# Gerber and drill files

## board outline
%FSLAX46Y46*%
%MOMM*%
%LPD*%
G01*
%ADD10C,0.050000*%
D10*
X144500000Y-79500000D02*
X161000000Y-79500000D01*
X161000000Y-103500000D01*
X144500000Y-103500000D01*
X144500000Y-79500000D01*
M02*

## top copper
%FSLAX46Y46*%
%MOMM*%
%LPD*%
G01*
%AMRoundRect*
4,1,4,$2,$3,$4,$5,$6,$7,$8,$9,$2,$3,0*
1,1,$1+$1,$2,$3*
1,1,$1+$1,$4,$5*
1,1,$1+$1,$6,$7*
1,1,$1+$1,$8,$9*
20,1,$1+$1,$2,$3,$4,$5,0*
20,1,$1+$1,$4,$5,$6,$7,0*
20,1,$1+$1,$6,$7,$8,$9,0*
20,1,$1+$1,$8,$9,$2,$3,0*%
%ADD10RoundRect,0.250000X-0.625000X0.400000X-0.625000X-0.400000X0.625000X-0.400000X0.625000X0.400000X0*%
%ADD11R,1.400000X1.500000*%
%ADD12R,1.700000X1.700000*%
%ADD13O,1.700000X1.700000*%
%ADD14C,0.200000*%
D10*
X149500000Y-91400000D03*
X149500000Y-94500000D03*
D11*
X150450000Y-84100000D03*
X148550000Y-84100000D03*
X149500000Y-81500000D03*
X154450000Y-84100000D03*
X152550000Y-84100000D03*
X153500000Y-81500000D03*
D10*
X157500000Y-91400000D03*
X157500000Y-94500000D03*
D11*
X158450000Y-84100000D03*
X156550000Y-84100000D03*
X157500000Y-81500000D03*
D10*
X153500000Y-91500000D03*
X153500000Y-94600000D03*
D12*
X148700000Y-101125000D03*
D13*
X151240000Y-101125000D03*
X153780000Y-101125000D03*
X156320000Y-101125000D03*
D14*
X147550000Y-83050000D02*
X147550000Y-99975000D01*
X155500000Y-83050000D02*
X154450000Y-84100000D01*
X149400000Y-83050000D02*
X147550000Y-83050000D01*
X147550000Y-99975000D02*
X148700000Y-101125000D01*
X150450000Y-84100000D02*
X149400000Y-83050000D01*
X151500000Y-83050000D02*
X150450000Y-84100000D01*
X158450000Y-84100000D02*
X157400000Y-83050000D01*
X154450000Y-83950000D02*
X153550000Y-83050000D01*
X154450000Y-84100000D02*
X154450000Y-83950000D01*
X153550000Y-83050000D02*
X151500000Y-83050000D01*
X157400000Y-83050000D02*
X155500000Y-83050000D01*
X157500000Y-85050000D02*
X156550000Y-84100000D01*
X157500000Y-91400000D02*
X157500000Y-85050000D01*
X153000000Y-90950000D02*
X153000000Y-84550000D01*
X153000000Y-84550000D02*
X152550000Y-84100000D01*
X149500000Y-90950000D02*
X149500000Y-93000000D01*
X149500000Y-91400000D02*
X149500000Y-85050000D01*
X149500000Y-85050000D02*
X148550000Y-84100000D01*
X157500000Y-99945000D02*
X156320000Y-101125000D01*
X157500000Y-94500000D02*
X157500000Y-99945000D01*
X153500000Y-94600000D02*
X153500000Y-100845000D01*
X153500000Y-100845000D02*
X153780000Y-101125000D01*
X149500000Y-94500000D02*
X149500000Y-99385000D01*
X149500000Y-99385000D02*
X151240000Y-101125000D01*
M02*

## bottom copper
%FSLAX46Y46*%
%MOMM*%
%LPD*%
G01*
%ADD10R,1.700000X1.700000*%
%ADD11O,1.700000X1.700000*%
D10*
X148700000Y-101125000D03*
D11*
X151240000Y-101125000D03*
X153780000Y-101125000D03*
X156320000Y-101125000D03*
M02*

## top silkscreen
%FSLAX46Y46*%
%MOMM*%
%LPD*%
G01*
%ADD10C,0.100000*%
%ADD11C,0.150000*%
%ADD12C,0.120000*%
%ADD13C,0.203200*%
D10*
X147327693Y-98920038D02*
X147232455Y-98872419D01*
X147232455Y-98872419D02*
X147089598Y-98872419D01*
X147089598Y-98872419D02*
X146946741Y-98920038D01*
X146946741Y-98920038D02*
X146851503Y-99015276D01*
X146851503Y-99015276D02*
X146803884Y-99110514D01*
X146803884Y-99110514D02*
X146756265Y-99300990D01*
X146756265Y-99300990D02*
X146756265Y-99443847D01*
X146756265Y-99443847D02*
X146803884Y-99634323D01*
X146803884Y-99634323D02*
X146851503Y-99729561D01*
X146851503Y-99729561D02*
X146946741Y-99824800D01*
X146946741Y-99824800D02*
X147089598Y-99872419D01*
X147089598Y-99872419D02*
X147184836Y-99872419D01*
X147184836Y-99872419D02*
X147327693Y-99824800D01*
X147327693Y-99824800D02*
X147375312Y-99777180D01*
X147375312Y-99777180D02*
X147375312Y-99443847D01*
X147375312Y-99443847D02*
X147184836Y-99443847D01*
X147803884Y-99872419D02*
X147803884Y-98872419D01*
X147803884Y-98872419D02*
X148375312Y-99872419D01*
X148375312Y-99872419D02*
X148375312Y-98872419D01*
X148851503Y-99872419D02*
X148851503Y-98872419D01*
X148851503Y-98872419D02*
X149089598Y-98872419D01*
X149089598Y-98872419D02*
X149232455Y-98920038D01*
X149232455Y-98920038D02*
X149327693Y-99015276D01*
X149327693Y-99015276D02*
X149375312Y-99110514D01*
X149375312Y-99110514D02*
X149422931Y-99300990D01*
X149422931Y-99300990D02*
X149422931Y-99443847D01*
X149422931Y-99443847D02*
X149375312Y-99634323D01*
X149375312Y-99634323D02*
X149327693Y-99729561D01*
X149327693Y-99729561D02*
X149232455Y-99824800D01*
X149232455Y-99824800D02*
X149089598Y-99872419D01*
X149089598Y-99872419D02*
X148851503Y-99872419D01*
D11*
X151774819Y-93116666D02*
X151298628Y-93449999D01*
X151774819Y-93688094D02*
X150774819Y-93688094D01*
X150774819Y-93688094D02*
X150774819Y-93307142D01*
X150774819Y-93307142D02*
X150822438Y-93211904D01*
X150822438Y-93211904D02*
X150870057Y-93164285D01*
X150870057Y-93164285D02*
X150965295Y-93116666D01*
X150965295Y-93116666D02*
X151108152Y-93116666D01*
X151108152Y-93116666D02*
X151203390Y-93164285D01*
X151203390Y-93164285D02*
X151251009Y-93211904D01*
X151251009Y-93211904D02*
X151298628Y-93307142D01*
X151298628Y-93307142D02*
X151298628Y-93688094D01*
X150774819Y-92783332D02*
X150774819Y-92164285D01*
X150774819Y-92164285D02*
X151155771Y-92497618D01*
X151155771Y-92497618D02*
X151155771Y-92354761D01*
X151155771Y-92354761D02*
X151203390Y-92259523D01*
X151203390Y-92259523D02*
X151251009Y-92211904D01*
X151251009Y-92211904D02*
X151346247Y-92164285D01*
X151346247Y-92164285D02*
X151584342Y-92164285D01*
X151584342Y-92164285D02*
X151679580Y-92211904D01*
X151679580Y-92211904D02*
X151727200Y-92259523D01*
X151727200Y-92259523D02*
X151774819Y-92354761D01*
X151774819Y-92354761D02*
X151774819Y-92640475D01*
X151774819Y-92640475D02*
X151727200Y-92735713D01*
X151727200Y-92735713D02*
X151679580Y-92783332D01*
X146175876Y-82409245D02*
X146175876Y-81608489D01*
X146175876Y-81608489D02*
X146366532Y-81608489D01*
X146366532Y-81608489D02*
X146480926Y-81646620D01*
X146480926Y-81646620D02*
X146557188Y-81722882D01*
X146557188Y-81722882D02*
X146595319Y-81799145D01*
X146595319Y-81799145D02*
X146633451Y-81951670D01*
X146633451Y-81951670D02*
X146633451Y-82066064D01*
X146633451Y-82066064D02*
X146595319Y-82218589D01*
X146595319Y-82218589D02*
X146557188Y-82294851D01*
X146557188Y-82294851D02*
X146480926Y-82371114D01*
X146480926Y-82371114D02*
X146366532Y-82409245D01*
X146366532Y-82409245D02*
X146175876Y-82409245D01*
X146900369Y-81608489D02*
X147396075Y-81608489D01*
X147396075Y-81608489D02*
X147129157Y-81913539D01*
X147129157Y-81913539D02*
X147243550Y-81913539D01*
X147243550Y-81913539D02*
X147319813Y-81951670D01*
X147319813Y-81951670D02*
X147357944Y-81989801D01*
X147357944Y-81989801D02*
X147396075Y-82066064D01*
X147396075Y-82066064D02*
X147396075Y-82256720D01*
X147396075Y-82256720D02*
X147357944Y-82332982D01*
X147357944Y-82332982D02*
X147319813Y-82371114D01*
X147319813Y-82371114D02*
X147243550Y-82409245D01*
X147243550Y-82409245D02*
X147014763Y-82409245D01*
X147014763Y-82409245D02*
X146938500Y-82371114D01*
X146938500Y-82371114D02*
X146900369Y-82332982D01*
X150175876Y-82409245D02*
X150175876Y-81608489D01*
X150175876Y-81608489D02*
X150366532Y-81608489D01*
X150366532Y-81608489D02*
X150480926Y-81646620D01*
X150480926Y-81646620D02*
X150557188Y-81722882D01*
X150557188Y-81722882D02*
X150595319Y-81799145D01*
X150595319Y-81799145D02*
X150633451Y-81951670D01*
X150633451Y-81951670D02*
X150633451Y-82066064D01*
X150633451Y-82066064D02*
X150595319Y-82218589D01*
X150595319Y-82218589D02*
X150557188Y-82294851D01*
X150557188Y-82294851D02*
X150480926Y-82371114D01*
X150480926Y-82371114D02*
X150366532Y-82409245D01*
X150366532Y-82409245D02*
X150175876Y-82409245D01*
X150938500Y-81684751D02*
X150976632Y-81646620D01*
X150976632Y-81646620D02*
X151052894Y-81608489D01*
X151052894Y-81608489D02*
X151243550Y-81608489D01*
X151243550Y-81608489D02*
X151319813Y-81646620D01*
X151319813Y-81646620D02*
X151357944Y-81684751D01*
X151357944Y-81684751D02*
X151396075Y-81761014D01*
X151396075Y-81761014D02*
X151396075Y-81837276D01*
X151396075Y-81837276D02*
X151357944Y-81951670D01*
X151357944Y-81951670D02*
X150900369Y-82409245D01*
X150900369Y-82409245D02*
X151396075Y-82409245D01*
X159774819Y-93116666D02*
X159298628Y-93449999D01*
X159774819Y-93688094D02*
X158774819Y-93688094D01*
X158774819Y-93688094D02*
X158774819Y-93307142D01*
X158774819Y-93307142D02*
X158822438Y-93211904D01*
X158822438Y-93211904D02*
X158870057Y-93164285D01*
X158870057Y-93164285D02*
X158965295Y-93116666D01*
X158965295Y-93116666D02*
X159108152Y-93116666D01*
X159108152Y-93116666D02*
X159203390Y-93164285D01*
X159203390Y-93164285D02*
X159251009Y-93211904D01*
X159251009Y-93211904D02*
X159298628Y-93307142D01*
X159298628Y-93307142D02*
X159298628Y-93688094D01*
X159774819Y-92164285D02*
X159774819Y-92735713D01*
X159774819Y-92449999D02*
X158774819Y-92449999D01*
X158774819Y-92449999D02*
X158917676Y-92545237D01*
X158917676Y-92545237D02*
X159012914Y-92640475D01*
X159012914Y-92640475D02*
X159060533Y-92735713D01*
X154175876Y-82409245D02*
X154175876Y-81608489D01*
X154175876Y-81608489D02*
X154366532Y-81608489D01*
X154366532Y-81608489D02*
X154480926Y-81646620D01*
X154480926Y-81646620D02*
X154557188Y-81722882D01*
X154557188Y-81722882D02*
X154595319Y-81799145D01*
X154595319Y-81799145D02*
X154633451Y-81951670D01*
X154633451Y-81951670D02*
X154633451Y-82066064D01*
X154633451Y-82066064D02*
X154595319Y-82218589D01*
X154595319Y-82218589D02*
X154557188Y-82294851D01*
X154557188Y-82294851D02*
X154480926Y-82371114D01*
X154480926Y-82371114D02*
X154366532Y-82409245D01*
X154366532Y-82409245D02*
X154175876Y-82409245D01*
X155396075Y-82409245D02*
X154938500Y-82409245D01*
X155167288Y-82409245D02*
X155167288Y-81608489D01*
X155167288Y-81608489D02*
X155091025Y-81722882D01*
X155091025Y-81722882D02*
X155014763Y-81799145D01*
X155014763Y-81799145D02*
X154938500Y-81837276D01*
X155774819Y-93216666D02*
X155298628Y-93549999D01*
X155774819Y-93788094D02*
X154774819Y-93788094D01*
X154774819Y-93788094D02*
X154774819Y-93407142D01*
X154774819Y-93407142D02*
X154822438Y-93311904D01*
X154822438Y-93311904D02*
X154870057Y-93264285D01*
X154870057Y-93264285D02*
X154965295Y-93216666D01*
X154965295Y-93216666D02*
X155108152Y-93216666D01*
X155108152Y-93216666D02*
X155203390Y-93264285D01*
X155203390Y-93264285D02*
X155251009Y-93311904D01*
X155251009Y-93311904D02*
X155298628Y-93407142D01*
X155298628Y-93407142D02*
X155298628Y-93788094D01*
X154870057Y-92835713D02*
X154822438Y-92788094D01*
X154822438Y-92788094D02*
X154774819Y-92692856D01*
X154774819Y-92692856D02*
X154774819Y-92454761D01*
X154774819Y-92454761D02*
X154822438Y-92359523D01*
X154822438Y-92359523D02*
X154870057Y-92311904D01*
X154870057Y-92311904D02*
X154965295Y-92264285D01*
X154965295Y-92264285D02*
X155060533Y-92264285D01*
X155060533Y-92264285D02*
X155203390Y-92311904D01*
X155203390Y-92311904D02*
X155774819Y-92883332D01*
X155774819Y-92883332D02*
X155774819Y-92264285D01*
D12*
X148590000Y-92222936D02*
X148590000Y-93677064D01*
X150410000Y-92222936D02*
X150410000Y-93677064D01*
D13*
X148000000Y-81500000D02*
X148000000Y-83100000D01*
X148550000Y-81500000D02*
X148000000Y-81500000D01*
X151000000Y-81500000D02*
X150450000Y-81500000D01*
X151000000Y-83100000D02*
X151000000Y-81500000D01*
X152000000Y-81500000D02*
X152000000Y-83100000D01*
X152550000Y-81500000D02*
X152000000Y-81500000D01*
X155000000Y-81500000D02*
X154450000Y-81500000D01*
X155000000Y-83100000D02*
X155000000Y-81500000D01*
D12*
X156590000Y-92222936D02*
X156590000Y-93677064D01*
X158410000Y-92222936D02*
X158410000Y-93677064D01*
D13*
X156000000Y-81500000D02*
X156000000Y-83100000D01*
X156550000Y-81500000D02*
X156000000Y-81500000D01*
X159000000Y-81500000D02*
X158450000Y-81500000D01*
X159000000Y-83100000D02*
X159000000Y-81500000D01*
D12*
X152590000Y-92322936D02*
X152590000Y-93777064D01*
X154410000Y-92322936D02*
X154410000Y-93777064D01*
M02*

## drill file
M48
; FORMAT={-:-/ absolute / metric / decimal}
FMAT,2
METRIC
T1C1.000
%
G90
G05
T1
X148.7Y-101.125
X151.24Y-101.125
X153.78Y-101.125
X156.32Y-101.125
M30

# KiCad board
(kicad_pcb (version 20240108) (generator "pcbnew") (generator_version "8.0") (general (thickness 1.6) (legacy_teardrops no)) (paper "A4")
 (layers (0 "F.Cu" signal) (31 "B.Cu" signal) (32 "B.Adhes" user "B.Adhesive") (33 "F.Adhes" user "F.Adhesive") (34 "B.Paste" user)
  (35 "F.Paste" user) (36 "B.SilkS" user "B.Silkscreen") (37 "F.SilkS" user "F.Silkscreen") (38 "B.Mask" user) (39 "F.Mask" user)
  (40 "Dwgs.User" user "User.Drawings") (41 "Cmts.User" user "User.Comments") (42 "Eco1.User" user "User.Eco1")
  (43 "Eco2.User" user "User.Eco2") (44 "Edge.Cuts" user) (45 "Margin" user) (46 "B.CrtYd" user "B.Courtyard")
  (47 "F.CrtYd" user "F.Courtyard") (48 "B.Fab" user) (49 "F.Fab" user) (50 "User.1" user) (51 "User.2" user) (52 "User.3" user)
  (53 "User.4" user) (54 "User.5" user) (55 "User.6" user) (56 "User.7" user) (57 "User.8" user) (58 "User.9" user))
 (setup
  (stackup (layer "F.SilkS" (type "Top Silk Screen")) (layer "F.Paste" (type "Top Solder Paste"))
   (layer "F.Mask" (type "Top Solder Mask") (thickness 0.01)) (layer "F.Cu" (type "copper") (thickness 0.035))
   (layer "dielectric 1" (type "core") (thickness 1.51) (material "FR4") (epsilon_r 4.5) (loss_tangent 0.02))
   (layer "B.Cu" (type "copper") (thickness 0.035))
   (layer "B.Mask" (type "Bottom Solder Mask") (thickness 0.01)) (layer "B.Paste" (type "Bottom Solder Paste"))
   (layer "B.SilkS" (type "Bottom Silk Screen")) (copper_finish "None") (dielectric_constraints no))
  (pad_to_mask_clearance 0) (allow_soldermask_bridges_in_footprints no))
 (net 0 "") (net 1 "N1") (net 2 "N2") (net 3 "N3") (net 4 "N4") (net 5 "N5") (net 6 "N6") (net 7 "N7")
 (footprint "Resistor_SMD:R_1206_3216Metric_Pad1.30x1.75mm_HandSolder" (layer "F.Cu") (at 149.5 92.95 -90)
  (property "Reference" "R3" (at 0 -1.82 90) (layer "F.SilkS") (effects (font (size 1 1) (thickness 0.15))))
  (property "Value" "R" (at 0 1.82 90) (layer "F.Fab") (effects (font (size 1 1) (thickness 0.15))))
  (fp_line (start -0.727064 0.91) (end 0.727064 0.91) (stroke (width 0.12) (type solid)) (layer "F.SilkS"))
  (fp_line (start -0.727064 -0.91) (end 0.727064 -0.91) (stroke (width 0.12) (type solid)) (layer "F.SilkS"))
  (pad "1" smd roundrect (at -1.55 0 270) (size 1.3 1.75) (layers "F.Cu" "F.Paste" "F.Mask") (roundrect_rratio 0.192308) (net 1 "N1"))
  (pad "2" smd roundrect (at 1.55 0 270) (size 1.3 1.75) (layers "F.Cu" "F.Paste" "F.Mask") (roundrect_rratio 0.192308) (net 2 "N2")))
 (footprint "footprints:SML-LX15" (layer "F.Cu") (at 149.5 83)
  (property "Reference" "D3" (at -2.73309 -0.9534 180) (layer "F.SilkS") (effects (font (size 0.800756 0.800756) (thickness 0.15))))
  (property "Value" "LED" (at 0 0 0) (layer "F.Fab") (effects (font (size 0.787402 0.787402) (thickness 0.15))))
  (fp_line (start -1.5 -1.5) (end -1.5 0.1) (stroke (width 0.2032) (type solid)) (layer "F.SilkS"))
  (fp_line (start -0.95 -1.5) (end -1.5 -1.5) (stroke (width 0.2032) (type solid)) (layer "F.SilkS"))
  (fp_line (start 1.5 -1.5) (end 0.95 -1.5) (stroke (width 0.2032) (type solid)) (layer "F.SilkS"))
  (fp_line (start 1.5 0.1) (end 1.5 -1.5) (stroke (width 0.2032) (type solid)) (layer "F.SilkS"))
  (pad "1" smd rect (at 0.95 1.1) (size 1.4 1.5) (layers "F.Cu" "F.Paste" "F.Mask") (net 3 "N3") (solder_mask_margin 0.102))
  (pad "2" smd rect (at -0.95 1.1) (size 1.4 1.5) (layers "F.Cu" "F.Paste" "F.Mask") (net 1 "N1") (solder_mask_margin 0.102))
  (pad "3" smd rect (at 0 -1.5) (size 1.4 1.5) (layers "F.Cu" "F.Paste" "F.Mask") (solder_mask_margin 0.102)))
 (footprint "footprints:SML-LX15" (layer "F.Cu") (at 153.5 83)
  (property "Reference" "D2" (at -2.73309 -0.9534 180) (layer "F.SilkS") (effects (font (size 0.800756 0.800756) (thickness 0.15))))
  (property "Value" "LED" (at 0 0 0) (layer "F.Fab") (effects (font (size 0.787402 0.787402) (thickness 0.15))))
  (fp_line (start -1.5 -1.5) (end -1.5 0.1) (stroke (width 0.2032) (type solid)) (layer "F.SilkS"))
  (fp_line (start -0.95 -1.5) (end -1.5 -1.5) (stroke (width 0.2032) (type solid)) (layer "F.SilkS"))
  (fp_line (start 1.5 -1.5) (end 0.95 -1.5) (stroke (width 0.2032) (type solid)) (layer "F.SilkS"))
  (fp_line (start 1.5 0.1) (end 1.5 -1.5) (stroke (width 0.2032) (type solid)) (layer "F.SilkS"))
  (pad "1" smd rect (at 0.95 1.1) (size 1.4 1.5) (layers "F.Cu" "F.Paste" "F.Mask") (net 3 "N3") (solder_mask_margin 0.102))
  (pad "2" smd rect (at -0.95 1.1) (size 1.4 1.5) (layers "F.Cu" "F.Paste" "F.Mask") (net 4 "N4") (solder_mask_margin 0.102))
  (pad "3" smd rect (at 0 -1.5) (size 1.4 1.5) (layers "F.Cu" "F.Paste" "F.Mask") (solder_mask_margin 0.102)))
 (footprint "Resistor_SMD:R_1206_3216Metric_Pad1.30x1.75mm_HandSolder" (layer "F.Cu") (at 157.5 92.95 -90)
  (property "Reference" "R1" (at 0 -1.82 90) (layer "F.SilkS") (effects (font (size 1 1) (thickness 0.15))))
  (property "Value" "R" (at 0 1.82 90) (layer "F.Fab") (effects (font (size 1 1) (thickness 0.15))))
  (fp_line (start -0.727064 0.91) (end 0.727064 0.91) (stroke (width 0.12) (type solid)) (layer "F.SilkS"))
  (fp_line (start -0.727064 -0.91) (end 0.727064 -0.91) (stroke (width 0.12) (type solid)) (layer "F.SilkS"))
  (pad "1" smd roundrect (at -1.55 0 270) (size 1.3 1.75) (layers "F.Cu" "F.Paste" "F.Mask") (roundrect_rratio 0.192308) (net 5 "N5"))
  (pad "2" smd roundrect (at 1.55 0 270) (size 1.3 1.75) (layers "F.Cu" "F.Paste" "F.Mask") (roundrect_rratio 0.192308) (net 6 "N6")))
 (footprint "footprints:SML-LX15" (layer "F.Cu") (at 157.5 83)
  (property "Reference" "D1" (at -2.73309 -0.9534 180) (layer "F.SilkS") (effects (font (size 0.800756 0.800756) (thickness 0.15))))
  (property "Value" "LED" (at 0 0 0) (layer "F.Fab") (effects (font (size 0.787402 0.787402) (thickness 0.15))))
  (fp_line (start -1.5 -1.5) (end -1.5 0.1) (stroke (width 0.2032) (type solid)) (layer "F.SilkS"))
  (fp_line (start -0.95 -1.5) (end -1.5 -1.5) (stroke (width 0.2032) (type solid)) (layer "F.SilkS"))
  (fp_line (start 1.5 -1.5) (end 0.95 -1.5) (stroke (width 0.2032) (type solid)) (layer "F.SilkS"))
  (fp_line (start 1.5 0.1) (end 1.5 -1.5) (stroke (width 0.2032) (type solid)) (layer "F.SilkS"))
  (pad "1" smd rect (at 0.95 1.1) (size 1.4 1.5) (layers "F.Cu" "F.Paste" "F.Mask") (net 3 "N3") (solder_mask_margin 0.102))
  (pad "2" smd rect (at -0.95 1.1) (size 1.4 1.5) (layers "F.Cu" "F.Paste" "F.Mask") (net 5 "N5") (solder_mask_margin 0.102))
  (pad "3" smd rect (at 0 -1.5) (size 1.4 1.5) (layers "F.Cu" "F.Paste" "F.Mask") (solder_mask_margin 0.102)))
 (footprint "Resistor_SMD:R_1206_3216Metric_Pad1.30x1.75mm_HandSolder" (layer "F.Cu") (at 153.5 93.05 -90)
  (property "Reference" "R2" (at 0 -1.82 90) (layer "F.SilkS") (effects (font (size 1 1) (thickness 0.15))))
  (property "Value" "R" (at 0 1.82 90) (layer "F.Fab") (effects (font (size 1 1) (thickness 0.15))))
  (fp_line (start -0.727064 0.91) (end 0.727064 0.91) (stroke (width 0.12) (type solid)) (layer "F.SilkS"))
  (fp_line (start -0.727064 -0.91) (end 0.727064 -0.91) (stroke (width 0.12) (type solid)) (layer "F.SilkS"))
  (pad "1" smd roundrect (at -1.55 0 270) (size 1.3 1.75) (layers "F.Cu" "F.Paste" "F.Mask") (roundrect_rratio 0.192308) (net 4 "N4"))
  (pad "2" smd roundrect (at 1.55 0 270) (size 1.3 1.75) (layers "F.Cu" "F.Paste" "F.Mask") (roundrect_rratio 0.192308) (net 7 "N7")))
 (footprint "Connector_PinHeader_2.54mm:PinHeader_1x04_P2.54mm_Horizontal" (layer "B.Cu") (at 148.7 101.125 -90)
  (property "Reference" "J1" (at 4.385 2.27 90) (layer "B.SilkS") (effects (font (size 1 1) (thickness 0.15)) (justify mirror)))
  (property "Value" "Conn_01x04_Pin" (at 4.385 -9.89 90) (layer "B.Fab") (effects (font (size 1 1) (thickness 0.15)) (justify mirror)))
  (pad "1" thru_hole rect (at 0 0 270) (size 1.7 1.7) (drill 1) (layers "*.Cu" "*.Mask") (remove_unused_layers no) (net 3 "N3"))
  (pad "2" thru_hole oval (at 0 -2.54 270) (size 1.7 1.7) (drill 1) (layers "*.Cu" "*.Mask") (remove_unused_layers no) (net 2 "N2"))
  (pad "3" thru_hole oval (at 0 -5.08 270) (size 1.7 1.7) (drill 1) (layers "*.Cu" "*.Mask") (remove_unused_layers no) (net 7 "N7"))
  (pad "4" thru_hole oval (at 0 -7.62 270) (size 1.7 1.7) (drill 1) (layers "*.Cu" "*.Mask") (remove_unused_layers no) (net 6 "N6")))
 (gr_rect (start 144.5 79.5) (end 161 103.5) (stroke (width 0.05) (type default)) (fill none) (layer "Edge.Cuts"))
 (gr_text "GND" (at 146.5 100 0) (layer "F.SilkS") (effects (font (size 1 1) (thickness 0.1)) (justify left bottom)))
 (segment (start 147.55 83.05) (end 147.55 99.975) (width 0.2) (layer "F.Cu") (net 3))
 (segment (start 155.5 83.05) (end 154.45 84.1) (width 0.2) (layer "F.Cu") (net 3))
 (segment (start 149.4 83.05) (end 147.55 83.05) (width 0.2) (layer "F.Cu") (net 3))
 (segment (start 147.55 99.975) (end 148.7 101.125) (width 0.2) (layer "F.Cu") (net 3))
 (segment (start 150.45 84.1) (end 149.4 83.05) (width 0.2) (layer "F.Cu") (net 3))
 (segment (start 151.5 83.05) (end 150.45 84.1) (width 0.2) (layer "F.Cu") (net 3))
 (segment (start 158.45 84.1) (end 157.4 83.05) (width 0.2) (layer "F.Cu") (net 3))
 (segment (start 154.45 83.95) (end 153.55 83.05) (width 0.2) (layer "F.Cu") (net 3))
 (segment (start 154.45 84.1) (end 154.45 83.95) (width 0.2) (layer "F.Cu") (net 3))
 (segment (start 153.55 83.05) (end 151.5 83.05) (width 0.2) (layer "F.Cu") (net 3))
 (segment (start 157.4 83.05) (end 155.5 83.05) (width 0.2) (layer "F.Cu") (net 3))
 (segment (start 157.5 85.05) (end 156.55 84.1) (width 0.2) (layer "F.Cu") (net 5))
 (segment (start 157.5 91.4) (end 157.5 85.05) (width 0.2) (layer "F.Cu") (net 5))
 (segment (start 153 90.95) (end 153 84.55) (width 0.2) (layer "F.Cu") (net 4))
 (segment (start 153 84.55) (end 152.55 84.1) (width 0.2) (layer "F.Cu") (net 4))
 (segment (start 149.5 90.95) (end 149.5 93) (width 0.2) (layer "F.Cu") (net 1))
 (segment (start 149.5 91.4) (end 149.5 85.05) (width 0.2) (layer "F.Cu") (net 1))
 (segment (start 149.5 85.05) (end 148.55 84.1) (width 0.2) (layer "F.Cu") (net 1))
 (segment (start 157.5 99.945) (end 156.32 101.125) (width 0.2) (layer "F.Cu") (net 6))
 (segment (start 157.5 94.5) (end 157.5 99.945) (width 0.2) (layer "F.Cu") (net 6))
 (segment (start 153.5 94.6) (end 153.5 100.845) (width 0.2) (layer "F.Cu") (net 7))
 (segment (start 153.5 100.845) (end 153.78 101.125) (width 0.2) (layer "F.Cu") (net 7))
 (segment (start 149.5 94.5) (end 149.5 99.385) (width 0.2) (layer "F.Cu") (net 2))
 (segment (start 149.5 99.385) (end 151.24 101.125) (width 0.2) (layer "F.Cu") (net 2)))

